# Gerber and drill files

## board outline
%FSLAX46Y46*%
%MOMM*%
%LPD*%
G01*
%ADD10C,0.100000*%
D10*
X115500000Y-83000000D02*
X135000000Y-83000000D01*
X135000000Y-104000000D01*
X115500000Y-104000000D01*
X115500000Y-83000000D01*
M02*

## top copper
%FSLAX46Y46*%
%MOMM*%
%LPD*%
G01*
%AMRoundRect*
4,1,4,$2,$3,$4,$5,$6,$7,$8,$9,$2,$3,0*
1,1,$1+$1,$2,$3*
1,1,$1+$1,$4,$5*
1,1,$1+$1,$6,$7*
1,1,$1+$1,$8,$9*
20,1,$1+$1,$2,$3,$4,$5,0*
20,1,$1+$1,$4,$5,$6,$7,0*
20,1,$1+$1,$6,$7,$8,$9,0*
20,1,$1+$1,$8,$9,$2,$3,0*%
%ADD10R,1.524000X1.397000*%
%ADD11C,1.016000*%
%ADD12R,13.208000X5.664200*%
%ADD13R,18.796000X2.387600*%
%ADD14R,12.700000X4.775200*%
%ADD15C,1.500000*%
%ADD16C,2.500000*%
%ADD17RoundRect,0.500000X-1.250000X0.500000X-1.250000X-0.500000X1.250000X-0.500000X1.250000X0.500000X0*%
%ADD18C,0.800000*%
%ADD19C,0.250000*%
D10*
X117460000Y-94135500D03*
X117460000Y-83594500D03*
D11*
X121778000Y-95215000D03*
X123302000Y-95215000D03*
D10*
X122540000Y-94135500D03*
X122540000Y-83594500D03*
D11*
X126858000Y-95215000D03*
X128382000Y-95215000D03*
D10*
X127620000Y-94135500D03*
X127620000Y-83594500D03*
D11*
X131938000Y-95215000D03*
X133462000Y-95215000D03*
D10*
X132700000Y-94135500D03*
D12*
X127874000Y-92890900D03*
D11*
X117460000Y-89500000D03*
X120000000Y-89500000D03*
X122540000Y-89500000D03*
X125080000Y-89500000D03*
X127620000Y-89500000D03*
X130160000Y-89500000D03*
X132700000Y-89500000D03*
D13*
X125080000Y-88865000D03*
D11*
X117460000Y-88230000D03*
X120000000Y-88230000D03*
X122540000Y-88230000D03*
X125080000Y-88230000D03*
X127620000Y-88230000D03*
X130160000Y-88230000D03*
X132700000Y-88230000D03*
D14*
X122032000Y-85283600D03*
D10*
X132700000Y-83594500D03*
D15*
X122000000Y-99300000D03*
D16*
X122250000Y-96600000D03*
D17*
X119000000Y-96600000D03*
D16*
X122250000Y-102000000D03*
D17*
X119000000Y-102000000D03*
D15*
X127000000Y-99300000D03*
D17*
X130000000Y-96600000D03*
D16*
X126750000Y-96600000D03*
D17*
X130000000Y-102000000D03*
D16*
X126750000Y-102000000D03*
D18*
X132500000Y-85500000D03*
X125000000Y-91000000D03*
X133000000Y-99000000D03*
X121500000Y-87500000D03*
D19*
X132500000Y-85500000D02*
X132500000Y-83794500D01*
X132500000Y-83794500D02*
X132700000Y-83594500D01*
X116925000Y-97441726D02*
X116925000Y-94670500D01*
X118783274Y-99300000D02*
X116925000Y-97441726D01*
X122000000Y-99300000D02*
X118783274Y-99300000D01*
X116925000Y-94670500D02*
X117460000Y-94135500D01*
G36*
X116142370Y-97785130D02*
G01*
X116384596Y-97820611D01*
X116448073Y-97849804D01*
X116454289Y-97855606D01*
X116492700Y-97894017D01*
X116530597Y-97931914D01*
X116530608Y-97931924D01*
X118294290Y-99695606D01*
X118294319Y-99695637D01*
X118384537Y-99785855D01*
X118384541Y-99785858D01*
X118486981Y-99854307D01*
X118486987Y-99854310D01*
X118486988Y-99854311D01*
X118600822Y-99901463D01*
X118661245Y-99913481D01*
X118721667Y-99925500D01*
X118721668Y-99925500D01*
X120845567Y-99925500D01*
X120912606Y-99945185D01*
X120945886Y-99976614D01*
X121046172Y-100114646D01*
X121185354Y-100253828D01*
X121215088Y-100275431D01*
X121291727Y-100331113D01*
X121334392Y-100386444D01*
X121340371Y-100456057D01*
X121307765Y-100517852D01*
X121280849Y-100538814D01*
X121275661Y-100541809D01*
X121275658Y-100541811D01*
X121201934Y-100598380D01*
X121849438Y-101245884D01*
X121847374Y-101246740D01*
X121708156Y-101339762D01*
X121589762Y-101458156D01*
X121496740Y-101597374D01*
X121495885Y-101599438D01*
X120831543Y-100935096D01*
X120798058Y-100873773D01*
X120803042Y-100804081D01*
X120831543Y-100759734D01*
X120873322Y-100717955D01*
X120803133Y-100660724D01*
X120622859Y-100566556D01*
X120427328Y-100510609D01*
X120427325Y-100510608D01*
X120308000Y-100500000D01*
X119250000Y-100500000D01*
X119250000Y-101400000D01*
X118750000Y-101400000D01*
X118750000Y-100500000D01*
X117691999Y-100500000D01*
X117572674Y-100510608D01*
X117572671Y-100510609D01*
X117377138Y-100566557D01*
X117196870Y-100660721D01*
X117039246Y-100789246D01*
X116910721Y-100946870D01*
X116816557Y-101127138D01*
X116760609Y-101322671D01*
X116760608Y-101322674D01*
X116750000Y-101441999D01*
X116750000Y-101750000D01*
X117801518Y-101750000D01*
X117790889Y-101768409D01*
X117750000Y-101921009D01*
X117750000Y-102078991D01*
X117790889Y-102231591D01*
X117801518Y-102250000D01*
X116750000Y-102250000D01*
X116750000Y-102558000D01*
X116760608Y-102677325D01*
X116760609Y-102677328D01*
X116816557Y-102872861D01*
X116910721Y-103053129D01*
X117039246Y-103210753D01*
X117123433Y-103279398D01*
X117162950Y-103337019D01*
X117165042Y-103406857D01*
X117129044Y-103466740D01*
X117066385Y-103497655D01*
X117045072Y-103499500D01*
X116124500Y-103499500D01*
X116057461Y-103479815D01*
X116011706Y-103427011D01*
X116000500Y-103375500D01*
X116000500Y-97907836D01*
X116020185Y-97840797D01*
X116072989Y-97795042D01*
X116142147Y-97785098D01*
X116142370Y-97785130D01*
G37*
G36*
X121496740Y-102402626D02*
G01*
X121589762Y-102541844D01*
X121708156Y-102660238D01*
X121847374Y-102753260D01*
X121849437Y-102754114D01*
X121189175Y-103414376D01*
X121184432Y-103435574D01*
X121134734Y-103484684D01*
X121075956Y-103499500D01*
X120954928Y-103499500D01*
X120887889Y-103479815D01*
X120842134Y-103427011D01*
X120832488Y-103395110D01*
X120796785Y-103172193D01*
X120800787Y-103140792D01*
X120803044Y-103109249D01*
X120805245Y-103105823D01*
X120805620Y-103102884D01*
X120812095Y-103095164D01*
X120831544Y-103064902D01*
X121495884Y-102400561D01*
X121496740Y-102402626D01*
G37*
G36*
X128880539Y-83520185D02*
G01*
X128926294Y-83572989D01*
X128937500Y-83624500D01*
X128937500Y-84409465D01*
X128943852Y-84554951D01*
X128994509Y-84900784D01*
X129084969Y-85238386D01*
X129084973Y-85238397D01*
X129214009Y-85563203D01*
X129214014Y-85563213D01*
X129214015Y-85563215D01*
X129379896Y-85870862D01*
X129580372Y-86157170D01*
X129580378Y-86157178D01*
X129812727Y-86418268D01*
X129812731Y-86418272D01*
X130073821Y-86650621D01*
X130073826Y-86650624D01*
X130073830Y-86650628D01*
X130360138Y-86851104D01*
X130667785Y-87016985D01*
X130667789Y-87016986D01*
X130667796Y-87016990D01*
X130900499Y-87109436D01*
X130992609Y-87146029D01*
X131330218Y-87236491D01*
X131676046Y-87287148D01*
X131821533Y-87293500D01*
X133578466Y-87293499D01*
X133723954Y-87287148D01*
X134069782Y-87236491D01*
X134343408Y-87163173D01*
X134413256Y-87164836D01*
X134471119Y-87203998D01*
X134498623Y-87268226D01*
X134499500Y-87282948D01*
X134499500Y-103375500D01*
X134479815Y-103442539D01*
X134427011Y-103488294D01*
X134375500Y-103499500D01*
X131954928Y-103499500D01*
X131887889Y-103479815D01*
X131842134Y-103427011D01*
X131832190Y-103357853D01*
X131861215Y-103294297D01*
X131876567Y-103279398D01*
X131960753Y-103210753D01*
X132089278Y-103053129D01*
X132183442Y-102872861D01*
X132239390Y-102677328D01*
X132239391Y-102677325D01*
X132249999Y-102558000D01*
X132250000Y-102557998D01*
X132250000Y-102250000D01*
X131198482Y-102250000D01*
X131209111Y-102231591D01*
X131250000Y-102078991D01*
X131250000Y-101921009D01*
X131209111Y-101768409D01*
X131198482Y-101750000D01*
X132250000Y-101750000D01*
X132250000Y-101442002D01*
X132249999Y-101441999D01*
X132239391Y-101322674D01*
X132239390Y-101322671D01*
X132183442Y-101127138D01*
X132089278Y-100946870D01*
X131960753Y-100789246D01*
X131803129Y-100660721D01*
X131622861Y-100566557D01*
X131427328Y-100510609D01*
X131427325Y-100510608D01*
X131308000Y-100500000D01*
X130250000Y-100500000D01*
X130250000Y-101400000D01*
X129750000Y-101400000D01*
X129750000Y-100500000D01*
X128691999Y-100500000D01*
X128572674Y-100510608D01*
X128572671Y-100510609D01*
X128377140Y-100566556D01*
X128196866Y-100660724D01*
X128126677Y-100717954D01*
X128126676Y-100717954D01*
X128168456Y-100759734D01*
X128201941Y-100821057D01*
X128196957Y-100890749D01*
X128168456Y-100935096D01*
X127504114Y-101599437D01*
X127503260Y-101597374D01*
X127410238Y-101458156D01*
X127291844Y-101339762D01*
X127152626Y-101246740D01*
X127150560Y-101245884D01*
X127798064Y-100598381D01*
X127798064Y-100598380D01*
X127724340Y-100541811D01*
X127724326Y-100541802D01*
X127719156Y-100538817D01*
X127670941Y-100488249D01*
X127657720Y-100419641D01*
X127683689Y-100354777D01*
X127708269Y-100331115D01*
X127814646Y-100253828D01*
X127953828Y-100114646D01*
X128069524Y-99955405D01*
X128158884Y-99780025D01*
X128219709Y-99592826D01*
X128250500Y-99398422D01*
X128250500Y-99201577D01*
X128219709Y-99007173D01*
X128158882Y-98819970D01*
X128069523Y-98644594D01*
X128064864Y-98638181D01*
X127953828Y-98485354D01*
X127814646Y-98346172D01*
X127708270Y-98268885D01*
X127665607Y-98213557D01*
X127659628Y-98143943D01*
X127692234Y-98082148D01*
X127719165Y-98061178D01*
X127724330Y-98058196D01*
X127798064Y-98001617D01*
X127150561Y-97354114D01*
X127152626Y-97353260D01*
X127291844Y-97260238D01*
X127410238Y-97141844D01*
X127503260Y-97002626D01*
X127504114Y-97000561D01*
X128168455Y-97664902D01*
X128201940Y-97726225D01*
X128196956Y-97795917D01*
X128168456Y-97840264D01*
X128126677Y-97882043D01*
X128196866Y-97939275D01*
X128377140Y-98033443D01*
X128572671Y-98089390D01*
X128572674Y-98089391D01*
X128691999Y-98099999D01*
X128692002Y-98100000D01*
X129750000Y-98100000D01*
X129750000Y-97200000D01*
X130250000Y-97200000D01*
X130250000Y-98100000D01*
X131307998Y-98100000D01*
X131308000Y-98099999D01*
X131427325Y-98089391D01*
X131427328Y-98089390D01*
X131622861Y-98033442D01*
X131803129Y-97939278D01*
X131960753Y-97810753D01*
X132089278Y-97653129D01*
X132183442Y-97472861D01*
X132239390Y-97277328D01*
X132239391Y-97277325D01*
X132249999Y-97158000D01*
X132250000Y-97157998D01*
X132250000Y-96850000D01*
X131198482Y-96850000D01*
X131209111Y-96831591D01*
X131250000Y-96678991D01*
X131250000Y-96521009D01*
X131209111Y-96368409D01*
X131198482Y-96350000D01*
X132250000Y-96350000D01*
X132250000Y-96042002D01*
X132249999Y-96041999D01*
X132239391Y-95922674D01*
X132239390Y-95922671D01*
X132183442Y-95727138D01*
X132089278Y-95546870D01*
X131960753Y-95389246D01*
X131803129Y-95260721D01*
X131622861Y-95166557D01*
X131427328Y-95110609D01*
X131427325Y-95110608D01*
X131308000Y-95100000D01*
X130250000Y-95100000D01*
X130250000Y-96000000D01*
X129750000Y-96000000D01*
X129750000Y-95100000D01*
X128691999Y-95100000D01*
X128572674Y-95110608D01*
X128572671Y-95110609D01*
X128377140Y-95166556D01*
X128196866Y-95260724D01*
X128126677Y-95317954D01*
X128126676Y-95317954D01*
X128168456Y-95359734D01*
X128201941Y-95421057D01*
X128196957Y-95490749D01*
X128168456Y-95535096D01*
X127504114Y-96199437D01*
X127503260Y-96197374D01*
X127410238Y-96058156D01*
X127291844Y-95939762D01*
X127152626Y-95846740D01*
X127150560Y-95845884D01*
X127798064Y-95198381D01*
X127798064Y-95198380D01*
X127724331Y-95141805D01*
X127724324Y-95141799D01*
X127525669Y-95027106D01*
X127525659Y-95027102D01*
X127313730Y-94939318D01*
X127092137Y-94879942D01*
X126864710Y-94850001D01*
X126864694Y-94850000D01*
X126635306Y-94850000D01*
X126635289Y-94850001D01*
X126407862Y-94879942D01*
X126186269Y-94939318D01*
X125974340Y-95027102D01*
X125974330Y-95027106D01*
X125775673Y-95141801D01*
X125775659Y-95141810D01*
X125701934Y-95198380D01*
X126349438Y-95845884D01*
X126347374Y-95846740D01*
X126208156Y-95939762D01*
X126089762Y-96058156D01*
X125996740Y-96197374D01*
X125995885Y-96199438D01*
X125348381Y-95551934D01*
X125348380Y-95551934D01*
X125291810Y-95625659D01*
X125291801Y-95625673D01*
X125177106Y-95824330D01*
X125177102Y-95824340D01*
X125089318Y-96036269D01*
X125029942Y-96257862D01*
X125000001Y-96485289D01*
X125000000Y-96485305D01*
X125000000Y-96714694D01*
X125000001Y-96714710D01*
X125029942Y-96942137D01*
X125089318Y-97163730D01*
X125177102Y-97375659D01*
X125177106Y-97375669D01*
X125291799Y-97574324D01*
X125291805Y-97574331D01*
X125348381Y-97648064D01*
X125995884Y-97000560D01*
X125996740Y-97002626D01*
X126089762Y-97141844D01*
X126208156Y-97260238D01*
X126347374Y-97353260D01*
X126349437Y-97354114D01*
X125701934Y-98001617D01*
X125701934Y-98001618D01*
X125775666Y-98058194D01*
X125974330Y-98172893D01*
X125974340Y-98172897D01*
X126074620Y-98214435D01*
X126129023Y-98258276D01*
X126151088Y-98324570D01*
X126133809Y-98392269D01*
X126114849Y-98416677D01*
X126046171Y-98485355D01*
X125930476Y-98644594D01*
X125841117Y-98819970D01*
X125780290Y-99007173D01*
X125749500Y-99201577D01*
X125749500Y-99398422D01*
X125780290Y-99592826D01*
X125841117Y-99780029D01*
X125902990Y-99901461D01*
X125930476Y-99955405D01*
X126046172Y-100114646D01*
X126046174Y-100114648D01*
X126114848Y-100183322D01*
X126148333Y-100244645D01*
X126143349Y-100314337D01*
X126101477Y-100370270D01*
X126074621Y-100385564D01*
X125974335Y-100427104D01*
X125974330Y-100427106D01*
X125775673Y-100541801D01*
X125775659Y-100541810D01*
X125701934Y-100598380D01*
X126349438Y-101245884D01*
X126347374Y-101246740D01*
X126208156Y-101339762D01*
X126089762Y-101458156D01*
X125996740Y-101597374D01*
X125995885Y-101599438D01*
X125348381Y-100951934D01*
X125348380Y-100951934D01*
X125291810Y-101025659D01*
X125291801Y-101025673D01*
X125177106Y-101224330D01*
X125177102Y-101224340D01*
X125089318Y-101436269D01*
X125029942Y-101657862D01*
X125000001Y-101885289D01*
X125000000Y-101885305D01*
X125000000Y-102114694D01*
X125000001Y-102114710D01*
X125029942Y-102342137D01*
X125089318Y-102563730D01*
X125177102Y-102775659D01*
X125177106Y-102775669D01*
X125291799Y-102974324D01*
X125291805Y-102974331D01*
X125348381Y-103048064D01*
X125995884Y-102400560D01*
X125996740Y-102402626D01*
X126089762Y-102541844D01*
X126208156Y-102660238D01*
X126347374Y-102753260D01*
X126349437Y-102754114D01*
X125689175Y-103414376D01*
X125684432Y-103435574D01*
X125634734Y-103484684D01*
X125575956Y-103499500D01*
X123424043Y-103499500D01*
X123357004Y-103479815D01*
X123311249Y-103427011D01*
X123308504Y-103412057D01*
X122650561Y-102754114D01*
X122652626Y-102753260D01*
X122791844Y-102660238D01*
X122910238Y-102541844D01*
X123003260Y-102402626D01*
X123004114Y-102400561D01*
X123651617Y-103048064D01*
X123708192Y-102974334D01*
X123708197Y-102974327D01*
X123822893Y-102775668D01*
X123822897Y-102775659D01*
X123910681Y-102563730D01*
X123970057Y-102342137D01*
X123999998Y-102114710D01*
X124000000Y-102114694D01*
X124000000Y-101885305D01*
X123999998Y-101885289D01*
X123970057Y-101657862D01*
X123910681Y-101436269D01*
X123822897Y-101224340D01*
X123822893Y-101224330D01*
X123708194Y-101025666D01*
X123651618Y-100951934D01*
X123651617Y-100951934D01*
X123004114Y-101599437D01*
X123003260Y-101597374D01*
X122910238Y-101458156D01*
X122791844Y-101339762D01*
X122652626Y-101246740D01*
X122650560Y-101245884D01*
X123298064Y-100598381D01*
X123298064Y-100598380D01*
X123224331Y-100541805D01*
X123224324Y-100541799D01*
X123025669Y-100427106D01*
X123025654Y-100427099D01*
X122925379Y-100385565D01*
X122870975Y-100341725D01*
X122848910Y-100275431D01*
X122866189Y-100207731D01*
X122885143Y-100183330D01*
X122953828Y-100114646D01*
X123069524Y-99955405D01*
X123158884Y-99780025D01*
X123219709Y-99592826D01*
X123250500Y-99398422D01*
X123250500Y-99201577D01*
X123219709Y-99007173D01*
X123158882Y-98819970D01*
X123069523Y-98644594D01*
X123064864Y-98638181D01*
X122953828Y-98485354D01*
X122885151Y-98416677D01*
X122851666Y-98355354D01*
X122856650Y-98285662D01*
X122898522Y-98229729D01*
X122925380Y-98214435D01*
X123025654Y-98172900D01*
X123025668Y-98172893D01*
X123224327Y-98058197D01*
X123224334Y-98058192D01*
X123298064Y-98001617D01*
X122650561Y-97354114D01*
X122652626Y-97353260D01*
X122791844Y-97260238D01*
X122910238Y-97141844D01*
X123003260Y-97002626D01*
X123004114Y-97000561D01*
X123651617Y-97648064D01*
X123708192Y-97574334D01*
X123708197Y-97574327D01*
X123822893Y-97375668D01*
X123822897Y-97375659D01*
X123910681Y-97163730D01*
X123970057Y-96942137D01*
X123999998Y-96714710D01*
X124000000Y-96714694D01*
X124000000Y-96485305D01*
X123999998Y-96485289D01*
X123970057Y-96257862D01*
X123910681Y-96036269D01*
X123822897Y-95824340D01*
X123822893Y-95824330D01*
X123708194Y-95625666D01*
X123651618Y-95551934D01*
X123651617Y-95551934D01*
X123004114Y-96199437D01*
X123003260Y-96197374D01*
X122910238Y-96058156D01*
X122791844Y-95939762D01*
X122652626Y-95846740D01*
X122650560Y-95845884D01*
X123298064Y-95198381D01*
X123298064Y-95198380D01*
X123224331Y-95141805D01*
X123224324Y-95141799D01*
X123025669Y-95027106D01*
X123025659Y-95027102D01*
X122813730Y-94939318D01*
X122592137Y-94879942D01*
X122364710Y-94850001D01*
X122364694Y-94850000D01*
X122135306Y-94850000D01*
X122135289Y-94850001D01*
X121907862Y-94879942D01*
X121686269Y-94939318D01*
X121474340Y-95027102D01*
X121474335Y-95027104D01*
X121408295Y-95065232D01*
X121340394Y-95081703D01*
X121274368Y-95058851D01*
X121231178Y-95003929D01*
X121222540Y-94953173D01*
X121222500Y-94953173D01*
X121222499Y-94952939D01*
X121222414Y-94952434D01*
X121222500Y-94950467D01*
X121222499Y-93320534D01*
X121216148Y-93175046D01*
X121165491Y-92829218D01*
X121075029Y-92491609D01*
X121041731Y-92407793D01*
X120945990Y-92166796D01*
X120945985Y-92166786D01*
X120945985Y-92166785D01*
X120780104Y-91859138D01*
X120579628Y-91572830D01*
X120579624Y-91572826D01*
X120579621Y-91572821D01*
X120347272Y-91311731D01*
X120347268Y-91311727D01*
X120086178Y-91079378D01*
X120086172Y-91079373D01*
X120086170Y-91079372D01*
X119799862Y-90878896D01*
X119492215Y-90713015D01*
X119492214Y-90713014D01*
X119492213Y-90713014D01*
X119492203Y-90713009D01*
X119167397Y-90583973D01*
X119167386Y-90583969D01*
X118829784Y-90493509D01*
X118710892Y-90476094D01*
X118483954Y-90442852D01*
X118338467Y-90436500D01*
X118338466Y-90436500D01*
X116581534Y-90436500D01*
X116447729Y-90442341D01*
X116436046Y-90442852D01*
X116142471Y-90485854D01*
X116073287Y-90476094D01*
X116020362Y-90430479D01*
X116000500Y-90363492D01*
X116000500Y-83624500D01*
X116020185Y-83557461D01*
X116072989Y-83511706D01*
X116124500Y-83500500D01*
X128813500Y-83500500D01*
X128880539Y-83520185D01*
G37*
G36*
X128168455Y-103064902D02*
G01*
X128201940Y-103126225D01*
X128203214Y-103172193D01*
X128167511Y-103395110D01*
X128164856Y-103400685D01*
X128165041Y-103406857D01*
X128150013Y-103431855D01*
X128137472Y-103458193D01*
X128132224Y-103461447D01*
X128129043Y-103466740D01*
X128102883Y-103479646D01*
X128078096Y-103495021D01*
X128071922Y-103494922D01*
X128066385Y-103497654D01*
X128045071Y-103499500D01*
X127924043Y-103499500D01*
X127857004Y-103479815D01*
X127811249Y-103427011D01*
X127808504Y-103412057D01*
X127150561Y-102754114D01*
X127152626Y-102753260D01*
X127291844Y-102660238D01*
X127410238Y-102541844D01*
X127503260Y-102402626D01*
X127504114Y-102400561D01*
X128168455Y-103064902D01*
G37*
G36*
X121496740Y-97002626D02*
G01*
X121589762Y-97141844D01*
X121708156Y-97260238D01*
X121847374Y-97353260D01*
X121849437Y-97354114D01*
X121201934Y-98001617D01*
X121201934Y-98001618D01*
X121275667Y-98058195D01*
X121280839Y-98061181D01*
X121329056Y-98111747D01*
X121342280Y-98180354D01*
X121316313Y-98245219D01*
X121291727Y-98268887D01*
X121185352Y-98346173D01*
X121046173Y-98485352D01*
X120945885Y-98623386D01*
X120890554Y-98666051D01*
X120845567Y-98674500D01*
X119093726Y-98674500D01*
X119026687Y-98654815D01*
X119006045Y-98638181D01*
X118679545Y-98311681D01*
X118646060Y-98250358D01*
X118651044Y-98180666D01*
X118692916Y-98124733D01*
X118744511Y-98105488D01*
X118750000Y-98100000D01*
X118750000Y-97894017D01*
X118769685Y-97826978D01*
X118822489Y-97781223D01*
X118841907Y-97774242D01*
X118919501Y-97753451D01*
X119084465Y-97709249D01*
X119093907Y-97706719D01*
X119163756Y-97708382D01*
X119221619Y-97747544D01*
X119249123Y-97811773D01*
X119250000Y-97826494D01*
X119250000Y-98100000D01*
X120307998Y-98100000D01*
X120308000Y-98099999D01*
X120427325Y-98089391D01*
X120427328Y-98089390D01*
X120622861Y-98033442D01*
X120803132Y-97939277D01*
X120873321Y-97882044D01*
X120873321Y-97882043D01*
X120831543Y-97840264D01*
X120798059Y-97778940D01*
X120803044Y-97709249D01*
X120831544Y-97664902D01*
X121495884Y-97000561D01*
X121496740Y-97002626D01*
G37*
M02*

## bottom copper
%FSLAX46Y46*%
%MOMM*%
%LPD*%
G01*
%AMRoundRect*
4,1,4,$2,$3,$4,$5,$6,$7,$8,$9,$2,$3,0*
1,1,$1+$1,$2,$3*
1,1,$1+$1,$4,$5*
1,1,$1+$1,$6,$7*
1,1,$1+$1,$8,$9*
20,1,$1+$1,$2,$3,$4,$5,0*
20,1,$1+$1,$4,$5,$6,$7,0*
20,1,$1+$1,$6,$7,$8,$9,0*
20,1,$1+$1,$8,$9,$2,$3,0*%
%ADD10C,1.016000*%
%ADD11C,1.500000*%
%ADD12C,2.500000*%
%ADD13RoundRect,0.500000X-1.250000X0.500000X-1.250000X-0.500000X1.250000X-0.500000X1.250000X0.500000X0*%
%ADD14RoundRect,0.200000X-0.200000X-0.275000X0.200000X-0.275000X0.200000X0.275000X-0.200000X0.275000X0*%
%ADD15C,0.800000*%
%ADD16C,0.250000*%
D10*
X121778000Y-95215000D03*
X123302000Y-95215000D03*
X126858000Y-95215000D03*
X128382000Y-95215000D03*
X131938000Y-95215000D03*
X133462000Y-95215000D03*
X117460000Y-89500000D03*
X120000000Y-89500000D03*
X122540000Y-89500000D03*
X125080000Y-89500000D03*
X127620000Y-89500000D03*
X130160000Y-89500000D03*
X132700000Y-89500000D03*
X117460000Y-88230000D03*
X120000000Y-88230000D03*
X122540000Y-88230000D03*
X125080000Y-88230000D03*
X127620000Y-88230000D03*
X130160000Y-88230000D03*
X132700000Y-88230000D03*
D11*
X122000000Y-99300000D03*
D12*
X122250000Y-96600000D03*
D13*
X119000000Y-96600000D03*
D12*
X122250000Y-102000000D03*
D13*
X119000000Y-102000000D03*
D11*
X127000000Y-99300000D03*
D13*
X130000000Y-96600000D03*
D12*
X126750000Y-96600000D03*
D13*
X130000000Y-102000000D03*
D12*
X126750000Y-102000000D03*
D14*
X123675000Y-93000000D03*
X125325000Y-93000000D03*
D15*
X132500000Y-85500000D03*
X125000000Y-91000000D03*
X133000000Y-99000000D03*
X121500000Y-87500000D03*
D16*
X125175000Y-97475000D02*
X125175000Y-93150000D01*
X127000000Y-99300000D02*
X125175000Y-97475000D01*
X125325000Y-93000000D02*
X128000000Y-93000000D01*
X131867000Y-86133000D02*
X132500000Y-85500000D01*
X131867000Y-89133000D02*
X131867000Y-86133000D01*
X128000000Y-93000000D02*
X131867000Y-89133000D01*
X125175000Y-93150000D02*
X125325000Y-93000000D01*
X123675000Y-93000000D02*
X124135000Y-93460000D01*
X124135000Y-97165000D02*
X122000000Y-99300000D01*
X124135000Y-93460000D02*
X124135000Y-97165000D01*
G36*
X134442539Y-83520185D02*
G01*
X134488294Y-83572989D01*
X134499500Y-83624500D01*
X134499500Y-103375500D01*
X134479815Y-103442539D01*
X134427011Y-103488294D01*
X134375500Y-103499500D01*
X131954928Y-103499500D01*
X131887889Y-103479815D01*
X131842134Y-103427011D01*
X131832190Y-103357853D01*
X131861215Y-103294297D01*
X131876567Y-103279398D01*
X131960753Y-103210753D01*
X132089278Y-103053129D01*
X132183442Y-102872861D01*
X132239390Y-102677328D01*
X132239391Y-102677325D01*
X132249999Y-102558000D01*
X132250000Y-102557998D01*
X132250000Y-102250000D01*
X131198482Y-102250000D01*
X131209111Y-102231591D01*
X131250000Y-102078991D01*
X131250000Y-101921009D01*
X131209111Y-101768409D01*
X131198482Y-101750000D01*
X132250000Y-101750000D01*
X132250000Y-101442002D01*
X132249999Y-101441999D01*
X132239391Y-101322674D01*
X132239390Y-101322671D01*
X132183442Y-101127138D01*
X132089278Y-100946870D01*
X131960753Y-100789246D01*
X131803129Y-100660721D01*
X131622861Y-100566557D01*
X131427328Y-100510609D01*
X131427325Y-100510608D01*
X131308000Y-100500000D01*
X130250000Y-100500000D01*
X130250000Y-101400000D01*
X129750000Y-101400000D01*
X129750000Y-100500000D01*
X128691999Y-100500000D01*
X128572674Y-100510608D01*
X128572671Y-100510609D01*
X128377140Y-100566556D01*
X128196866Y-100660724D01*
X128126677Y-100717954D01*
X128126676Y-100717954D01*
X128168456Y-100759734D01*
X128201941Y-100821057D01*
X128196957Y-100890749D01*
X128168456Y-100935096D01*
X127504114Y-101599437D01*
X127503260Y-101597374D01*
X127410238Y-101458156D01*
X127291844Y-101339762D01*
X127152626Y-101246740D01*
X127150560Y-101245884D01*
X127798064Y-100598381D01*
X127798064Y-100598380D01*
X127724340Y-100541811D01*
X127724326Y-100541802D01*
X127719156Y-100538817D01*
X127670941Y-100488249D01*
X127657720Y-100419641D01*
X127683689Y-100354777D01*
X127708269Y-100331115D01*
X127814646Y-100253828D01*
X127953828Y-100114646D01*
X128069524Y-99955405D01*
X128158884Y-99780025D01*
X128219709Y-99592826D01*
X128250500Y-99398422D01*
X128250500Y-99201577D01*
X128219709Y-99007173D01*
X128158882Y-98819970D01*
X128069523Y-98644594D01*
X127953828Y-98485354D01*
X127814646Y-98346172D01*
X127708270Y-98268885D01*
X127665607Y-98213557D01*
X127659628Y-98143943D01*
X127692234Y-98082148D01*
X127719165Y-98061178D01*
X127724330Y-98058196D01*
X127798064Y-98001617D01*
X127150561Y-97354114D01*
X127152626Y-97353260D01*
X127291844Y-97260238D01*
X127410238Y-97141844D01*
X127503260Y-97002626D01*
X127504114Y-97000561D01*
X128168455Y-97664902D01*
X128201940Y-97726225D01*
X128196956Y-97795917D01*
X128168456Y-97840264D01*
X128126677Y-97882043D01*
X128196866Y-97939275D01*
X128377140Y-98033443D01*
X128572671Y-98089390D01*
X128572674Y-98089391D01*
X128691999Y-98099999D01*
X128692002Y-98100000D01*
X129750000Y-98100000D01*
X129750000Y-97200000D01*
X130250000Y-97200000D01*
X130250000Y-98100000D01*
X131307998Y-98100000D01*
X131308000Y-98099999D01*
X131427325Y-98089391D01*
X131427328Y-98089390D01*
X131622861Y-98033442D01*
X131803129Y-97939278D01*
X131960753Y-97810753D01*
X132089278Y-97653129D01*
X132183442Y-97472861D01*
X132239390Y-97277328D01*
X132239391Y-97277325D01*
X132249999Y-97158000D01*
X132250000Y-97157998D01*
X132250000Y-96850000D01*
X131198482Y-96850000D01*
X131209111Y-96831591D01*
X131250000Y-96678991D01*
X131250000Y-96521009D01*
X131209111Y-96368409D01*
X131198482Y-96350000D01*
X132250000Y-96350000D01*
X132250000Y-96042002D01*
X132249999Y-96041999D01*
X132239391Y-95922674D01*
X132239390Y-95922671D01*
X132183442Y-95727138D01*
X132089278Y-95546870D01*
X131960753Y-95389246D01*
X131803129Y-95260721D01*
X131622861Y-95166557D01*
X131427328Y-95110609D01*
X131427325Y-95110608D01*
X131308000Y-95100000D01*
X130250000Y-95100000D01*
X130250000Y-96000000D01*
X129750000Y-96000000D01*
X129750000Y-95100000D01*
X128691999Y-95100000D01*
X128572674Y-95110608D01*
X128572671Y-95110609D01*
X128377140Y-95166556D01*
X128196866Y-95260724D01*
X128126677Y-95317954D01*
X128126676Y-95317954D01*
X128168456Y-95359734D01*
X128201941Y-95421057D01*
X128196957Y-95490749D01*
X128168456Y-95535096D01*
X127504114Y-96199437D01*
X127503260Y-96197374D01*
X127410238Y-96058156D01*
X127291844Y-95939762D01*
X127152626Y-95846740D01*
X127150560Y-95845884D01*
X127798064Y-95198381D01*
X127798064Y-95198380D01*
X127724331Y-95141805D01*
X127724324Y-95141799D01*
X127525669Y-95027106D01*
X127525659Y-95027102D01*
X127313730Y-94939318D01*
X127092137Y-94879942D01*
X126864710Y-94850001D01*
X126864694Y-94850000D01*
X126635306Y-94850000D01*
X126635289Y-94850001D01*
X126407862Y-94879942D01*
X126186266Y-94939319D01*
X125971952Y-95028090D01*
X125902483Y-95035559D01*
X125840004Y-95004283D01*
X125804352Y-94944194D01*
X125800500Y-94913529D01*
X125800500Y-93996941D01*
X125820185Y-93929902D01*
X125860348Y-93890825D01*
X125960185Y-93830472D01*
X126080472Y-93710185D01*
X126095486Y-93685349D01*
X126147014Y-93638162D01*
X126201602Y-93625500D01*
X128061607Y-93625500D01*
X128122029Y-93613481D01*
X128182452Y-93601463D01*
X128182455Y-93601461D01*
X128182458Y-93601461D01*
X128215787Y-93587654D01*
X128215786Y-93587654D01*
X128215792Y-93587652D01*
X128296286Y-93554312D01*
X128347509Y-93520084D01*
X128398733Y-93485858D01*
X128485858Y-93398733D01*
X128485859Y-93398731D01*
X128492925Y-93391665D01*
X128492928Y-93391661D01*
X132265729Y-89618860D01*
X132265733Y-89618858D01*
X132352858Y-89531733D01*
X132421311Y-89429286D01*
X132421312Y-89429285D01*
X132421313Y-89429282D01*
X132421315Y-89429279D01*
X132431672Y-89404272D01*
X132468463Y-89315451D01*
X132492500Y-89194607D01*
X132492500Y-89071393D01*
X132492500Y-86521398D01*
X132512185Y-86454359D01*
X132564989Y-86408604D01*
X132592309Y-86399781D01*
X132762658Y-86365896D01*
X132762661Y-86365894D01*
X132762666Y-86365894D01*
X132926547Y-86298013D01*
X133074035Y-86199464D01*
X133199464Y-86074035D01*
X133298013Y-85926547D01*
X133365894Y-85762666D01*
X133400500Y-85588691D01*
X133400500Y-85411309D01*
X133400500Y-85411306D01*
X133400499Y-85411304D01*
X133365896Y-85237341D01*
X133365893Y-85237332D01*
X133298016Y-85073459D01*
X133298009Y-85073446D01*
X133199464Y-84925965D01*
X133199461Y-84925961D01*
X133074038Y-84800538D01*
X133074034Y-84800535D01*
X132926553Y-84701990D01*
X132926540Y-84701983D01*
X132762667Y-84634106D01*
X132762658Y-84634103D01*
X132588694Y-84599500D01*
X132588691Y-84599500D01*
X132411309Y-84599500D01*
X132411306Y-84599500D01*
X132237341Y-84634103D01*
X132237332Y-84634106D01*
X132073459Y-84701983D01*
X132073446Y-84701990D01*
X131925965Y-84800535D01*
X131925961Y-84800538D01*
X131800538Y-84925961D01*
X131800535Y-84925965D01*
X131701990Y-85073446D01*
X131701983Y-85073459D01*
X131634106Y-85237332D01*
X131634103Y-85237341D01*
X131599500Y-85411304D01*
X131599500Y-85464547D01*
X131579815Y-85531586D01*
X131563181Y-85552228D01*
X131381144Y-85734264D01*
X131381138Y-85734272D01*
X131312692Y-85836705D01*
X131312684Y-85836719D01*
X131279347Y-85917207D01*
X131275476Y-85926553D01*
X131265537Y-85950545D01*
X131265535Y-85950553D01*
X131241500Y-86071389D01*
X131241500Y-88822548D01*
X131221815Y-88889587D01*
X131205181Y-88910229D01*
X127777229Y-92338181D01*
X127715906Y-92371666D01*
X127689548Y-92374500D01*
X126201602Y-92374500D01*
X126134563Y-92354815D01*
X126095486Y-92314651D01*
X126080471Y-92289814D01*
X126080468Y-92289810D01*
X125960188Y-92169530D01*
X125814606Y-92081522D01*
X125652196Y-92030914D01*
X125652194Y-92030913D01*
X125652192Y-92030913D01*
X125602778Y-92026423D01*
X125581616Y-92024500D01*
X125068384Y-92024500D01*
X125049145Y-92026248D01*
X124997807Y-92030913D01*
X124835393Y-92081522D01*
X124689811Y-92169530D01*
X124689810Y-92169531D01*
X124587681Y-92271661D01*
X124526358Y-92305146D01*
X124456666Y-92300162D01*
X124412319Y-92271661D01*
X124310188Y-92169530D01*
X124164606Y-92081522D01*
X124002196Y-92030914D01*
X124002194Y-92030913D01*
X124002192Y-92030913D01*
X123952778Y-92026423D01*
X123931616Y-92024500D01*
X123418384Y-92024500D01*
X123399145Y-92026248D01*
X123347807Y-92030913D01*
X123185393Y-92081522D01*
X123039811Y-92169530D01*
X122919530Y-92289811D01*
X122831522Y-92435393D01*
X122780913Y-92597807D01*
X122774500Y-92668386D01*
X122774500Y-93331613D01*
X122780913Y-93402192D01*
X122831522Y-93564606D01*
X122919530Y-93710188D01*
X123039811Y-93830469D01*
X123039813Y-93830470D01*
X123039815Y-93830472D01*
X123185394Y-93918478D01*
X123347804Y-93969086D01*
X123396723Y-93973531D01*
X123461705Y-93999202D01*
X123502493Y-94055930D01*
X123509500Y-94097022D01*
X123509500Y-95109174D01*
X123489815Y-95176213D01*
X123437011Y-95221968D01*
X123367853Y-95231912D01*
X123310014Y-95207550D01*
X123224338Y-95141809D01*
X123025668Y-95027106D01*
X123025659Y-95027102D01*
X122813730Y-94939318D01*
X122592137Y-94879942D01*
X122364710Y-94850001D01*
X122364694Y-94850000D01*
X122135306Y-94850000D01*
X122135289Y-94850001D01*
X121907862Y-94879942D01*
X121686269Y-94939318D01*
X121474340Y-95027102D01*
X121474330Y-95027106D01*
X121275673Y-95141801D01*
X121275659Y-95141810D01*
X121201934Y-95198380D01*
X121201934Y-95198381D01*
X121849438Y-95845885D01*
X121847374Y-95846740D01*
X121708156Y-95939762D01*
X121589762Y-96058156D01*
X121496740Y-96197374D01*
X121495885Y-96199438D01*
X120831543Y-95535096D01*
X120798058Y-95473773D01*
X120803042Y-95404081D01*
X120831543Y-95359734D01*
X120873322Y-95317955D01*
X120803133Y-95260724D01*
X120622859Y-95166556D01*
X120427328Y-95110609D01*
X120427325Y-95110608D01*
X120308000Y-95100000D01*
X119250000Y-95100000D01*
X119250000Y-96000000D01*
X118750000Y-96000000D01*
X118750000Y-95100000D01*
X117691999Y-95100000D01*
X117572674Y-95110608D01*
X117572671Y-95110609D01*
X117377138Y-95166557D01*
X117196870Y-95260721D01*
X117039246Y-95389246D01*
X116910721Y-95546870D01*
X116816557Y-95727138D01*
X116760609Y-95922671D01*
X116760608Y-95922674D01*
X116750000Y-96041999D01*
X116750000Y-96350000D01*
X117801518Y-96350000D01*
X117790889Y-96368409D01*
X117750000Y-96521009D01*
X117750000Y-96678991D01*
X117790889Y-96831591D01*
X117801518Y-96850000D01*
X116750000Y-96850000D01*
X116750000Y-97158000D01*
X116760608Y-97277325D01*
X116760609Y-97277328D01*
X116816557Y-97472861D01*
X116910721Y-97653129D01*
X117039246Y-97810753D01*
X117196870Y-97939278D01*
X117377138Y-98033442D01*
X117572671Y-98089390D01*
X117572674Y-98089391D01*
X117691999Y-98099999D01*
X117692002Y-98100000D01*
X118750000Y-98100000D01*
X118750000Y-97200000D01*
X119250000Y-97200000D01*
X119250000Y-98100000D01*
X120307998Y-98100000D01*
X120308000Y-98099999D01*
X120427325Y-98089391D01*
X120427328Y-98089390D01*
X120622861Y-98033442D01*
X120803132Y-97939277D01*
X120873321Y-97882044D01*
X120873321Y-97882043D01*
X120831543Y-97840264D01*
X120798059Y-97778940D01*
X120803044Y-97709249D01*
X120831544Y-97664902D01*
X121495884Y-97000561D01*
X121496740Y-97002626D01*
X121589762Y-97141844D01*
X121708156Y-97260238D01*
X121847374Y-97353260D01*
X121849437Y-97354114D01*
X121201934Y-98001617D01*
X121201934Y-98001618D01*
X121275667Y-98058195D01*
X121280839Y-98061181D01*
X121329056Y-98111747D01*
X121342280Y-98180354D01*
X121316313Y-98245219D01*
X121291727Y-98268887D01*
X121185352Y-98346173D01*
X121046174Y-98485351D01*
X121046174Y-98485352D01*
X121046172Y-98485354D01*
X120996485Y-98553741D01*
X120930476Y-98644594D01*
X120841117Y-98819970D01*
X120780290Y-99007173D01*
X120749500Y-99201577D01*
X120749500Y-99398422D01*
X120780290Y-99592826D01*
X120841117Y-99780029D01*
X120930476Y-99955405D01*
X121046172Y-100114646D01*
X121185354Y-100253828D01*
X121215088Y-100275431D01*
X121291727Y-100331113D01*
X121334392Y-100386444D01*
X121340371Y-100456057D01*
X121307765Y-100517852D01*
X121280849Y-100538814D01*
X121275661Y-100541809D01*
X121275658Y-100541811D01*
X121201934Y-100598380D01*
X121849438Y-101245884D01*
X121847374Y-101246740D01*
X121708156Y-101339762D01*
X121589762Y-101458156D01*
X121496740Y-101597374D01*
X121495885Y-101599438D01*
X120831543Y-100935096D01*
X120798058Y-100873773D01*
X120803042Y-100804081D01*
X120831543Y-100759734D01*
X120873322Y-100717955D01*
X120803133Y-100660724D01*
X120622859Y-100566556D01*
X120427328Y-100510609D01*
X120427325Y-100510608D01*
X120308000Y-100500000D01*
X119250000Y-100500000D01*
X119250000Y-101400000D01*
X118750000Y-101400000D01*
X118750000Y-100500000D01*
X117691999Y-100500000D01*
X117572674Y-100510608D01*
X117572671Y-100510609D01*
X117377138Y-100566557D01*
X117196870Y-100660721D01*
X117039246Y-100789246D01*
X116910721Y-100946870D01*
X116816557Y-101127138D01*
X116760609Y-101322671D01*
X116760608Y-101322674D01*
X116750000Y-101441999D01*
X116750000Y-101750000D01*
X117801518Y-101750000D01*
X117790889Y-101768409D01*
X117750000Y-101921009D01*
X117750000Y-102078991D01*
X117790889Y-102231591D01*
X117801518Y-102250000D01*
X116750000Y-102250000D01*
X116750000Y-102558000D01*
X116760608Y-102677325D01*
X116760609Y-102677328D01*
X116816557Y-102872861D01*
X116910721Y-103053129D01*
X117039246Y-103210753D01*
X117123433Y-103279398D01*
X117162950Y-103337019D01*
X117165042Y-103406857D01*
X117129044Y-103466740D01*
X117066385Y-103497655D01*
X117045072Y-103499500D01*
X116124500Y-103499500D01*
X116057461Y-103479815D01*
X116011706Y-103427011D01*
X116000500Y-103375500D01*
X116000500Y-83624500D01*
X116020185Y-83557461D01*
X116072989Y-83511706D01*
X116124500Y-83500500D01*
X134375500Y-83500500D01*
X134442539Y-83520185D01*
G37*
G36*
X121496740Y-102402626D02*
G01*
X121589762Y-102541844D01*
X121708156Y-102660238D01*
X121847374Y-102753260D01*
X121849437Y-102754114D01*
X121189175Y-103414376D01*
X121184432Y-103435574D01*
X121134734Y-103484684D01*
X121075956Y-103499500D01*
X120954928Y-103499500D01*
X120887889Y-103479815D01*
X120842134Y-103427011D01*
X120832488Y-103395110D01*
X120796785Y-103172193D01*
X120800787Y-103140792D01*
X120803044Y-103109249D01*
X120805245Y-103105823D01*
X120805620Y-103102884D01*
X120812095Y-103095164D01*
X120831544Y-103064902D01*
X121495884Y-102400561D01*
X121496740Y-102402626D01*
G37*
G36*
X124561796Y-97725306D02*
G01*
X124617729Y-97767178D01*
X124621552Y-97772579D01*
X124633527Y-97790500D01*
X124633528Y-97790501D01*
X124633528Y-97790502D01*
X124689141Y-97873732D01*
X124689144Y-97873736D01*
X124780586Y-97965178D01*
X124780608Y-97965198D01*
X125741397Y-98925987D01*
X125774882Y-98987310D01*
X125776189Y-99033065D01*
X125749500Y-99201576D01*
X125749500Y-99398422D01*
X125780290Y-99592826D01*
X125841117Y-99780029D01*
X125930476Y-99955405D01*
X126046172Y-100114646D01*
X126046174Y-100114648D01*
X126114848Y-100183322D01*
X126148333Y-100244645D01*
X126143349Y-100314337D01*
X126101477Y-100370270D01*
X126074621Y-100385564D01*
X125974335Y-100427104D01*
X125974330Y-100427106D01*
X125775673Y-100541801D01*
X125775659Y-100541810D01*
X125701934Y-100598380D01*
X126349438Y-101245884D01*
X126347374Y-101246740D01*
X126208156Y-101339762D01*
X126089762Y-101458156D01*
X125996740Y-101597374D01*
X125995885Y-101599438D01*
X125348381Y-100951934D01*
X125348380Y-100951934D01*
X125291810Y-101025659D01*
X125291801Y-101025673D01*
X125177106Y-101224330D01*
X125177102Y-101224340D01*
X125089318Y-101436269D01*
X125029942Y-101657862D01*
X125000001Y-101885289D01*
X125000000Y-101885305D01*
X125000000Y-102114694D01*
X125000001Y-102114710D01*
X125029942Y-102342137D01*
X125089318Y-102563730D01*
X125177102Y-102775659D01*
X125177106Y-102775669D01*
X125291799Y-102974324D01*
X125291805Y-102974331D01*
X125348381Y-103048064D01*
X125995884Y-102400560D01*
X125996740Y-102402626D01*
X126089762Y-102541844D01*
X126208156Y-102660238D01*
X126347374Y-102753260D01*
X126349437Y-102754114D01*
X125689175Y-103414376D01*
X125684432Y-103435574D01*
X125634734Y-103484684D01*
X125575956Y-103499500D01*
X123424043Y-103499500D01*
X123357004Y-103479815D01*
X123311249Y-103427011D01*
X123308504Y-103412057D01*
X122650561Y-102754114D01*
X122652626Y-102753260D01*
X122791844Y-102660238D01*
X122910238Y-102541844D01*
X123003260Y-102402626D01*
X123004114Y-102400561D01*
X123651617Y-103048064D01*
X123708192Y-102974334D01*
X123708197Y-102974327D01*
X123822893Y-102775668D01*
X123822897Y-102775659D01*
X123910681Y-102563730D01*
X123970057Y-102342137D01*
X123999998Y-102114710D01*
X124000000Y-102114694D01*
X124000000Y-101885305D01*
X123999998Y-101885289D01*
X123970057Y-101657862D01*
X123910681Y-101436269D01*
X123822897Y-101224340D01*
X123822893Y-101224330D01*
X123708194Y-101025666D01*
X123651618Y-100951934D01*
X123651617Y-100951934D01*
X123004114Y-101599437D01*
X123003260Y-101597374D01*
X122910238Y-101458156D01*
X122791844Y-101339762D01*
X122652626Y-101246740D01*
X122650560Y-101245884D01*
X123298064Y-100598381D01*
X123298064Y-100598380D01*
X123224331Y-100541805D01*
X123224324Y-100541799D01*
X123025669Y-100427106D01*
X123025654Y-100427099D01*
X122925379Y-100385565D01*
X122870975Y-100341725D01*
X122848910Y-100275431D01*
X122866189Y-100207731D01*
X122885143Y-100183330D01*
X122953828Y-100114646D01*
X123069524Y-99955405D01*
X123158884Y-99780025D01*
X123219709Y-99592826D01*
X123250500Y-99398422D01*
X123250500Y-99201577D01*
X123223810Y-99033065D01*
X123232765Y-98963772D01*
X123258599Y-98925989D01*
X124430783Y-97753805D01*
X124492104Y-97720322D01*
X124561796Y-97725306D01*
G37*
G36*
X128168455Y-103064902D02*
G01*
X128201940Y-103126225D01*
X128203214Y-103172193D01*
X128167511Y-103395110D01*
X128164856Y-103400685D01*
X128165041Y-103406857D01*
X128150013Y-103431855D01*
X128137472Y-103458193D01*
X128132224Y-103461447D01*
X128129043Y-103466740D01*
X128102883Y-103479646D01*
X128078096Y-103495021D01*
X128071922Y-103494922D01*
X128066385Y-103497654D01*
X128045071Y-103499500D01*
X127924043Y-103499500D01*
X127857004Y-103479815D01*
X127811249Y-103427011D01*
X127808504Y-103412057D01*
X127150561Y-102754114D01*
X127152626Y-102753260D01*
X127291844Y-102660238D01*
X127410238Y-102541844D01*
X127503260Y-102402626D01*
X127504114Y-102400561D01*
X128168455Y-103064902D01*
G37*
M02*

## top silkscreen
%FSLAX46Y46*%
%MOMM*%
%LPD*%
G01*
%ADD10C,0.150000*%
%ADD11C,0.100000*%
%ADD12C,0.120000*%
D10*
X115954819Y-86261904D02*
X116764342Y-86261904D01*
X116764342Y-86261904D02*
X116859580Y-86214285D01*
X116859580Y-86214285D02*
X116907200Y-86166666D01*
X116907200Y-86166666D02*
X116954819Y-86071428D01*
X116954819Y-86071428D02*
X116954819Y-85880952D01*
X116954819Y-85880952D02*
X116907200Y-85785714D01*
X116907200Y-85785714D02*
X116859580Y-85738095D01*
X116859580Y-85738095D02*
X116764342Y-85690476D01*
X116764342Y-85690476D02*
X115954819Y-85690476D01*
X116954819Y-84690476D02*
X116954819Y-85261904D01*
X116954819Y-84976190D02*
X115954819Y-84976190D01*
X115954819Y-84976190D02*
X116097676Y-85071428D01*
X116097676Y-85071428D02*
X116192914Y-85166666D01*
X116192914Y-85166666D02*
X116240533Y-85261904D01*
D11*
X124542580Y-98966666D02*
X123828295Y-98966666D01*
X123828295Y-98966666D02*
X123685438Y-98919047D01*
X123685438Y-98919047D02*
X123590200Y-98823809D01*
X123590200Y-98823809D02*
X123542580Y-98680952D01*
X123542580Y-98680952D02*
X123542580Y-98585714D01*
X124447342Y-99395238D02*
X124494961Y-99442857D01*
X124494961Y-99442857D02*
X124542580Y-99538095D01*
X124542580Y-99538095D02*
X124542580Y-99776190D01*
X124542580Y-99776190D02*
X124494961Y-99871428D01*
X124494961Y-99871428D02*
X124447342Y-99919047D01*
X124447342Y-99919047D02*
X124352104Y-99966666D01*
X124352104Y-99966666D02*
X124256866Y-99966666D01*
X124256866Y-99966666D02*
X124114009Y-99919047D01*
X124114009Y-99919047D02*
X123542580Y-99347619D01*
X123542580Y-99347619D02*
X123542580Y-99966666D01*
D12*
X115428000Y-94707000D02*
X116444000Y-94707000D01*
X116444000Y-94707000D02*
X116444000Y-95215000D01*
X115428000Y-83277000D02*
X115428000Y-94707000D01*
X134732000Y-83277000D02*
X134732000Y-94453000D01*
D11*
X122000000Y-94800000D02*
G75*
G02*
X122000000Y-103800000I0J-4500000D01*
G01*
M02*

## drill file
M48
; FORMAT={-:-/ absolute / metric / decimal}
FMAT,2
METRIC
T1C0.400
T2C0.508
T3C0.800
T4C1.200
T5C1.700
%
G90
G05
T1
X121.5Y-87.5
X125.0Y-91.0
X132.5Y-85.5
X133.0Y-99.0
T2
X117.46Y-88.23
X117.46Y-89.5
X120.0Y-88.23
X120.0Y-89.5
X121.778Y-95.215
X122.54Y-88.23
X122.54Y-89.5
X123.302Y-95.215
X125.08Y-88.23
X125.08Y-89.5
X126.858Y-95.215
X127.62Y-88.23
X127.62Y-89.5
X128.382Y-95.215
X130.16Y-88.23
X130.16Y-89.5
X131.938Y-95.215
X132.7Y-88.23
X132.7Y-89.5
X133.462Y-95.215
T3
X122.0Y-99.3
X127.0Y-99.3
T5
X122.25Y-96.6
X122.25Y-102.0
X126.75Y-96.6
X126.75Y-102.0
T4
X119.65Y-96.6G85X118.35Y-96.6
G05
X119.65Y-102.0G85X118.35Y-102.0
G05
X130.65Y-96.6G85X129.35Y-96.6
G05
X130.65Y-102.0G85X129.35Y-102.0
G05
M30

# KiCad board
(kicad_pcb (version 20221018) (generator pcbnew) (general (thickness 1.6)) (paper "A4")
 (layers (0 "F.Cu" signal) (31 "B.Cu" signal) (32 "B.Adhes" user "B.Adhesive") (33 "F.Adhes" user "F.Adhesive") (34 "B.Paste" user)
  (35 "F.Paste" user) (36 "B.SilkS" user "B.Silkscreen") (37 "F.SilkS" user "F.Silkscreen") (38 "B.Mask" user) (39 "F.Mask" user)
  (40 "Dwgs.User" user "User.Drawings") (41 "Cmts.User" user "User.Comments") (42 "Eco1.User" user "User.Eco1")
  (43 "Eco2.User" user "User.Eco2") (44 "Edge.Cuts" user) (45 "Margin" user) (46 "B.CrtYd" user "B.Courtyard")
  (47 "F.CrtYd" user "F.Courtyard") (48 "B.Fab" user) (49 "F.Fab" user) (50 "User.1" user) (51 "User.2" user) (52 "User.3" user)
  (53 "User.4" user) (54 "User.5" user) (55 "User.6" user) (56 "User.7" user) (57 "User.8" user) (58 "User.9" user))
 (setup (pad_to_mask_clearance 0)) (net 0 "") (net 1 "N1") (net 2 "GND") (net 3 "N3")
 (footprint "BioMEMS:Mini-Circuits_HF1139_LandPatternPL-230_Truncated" (layer "F.Cu") (at 125.08 88.865 90)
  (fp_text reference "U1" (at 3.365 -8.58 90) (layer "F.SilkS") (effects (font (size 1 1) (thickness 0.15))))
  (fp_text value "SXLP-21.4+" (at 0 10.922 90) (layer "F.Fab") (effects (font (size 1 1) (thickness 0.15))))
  (fp_line (start -5.842 -9.652) (end -5.842 -8.636) (stroke (width 0.12) (type solid)) (layer "F.SilkS"))
  (fp_line (start -5.842 -8.636) (end -6.35 -8.636) (stroke (width 0.12) (type solid)) (layer "F.SilkS"))
  (fp_line (start 5.588 -9.652) (end -5.842 -9.652) (stroke (width 0.12) (type solid)) (layer "F.SilkS"))
  (fp_line (start 5.588 9.652) (end -5.588 9.652) (stroke (width 0.12) (type solid)) (layer "F.SilkS"))
  (pad "1" smd rect (at -5.2705 -7.62) (size 1.524 1.397) (layers "F.Cu" "F.Paste" "F.Mask") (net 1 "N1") (clearance 3))
  (pad "2" smd rect (at 5.2705 -7.62) (size 1.524 1.397) (layers "F.Cu" "F.Paste" "F.Mask") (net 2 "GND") (zone_connect 2))
  (pad "3" thru_hole circle (at -6.35 -3.302) (size 1.016 1.016) (drill 0.508) (layers "*.Cu") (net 2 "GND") (zone_connect 2))
  (pad "3" thru_hole circle (at -6.35 -1.778) (size 1.016 1.016) (drill 0.508) (layers "*.Cu") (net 2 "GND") (zone_connect 2))
  (pad "3" smd rect (at -5.2705 -2.54) (size 1.524 1.397) (layers "F.Cu" "F.Paste" "F.Mask") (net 2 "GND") (zone_connect 2))
  (pad "4" smd rect (at 5.2705 -2.54) (size 1.524 1.397) (layers "F.Cu" "F.Paste" "F.Mask") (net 2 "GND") (zone_connect 2))
  (pad "5" thru_hole circle (at -6.35 1.778) (size 1.016 1.016) (drill 0.508) (layers "*.Cu") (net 2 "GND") (zone_connect 2))
  (pad "5" thru_hole circle (at -6.35 3.302) (size 1.016 1.016) (drill 0.508) (layers "*.Cu") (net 2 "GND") (zone_connect 2))
  (pad "5" smd rect (at -5.2705 2.54) (size 1.524 1.397) (layers "F.Cu" "F.Paste" "F.Mask") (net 2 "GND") (zone_connect 2))
  (pad "6" smd rect (at 5.2705 2.54) (size 1.524 1.397) (layers "F.Cu" "F.Paste" "F.Mask") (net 2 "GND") (zone_connect 2))
  (pad "7" thru_hole circle (at -6.35 6.858) (size 1.016 1.016) (drill 0.508) (layers "*.Cu") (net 2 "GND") (zone_connect 2))
  (pad "7" thru_hole circle (at -6.35 8.382) (size 1.016 1.016) (drill 0.508) (layers "*.Cu") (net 2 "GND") (zone_connect 2))
  (pad "7" smd rect (at -5.2705 7.62) (size 1.524 1.397) (layers "F.Cu" "F.Paste" "F.Mask") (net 2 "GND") (zone_connect 2))
  (pad "7" smd rect (at -4.0259 2.794) (size 13.208 5.6642) (layers "F.Cu") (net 2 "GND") (zone_connect 2))
  (pad "7" thru_hole circle (at -0.635 -7.62) (size 1.016 1.016) (drill 0.508) (layers "*.Cu") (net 2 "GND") (zone_connect 2))
  (pad "7" thru_hole circle (at -0.635 -5.08) (size 1.016 1.016) (drill 0.508) (layers "*.Cu") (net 2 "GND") (zone_connect 2))
  (pad "7" thru_hole circle (at -0.635 -2.54) (size 1.016 1.016) (drill 0.508) (layers "*.Cu") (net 2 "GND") (zone_connect 2))
  (pad "7" thru_hole circle (at -0.635 0) (size 1.016 1.016) (drill 0.508) (layers "*.Cu") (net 2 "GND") (zone_connect 2))
  (pad "7" thru_hole circle (at -0.635 2.54) (size 1.016 1.016) (drill 0.508) (layers "*.Cu") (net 2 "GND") (zone_connect 2))
  (pad "7" thru_hole circle (at -0.635 5.08) (size 1.016 1.016) (drill 0.508) (layers "*.Cu") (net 2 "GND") (zone_connect 2))
  (pad "7" thru_hole circle (at -0.635 7.62) (size 1.016 1.016) (drill 0.508) (layers "*.Cu") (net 2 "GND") (zone_connect 2))
  (pad "7" smd rect (at 0 0) (size 18.796 2.3876) (layers "F.Cu") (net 2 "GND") (zone_connect 2))
  (pad "7" thru_hole circle (at 0.635 -7.62) (size 1.016 1.016) (drill 0.508) (layers "*.Cu") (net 2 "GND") (zone_connect 2))
  (pad "7" thru_hole circle (at 0.635 -5.08) (size 1.016 1.016) (drill 0.508) (layers "*.Cu") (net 2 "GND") (zone_connect 2))
  (pad "7" thru_hole circle (at 0.635 -2.54) (size 1.016 1.016) (drill 0.508) (layers "*.Cu") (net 2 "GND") (zone_connect 2))
  (pad "7" thru_hole circle (at 0.635 0) (size 1.016 1.016) (drill 0.508) (layers "*.Cu") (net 2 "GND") (zone_connect 2))
  (pad "7" thru_hole circle (at 0.635 2.54) (size 1.016 1.016) (drill 0.508) (layers "*.Cu") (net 2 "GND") (zone_connect 2))
  (pad "7" thru_hole circle (at 0.635 5.08) (size 1.016 1.016) (drill 0.508) (layers "*.Cu") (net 2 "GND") (zone_connect 2))
  (pad "7" thru_hole circle (at 0.635 7.62) (size 1.016 1.016) (drill 0.508) (layers "*.Cu") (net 2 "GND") (zone_connect 2))
  (pad "7" smd rect (at 3.5814 -3.048) (size 12.7 4.7752) (layers "F.Cu") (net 2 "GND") (zone_connect 2))
  (pad "8" smd rect (at 5.2705 7.62) (size 1.524 1.397) (layers "F.Cu" "F.Paste" "F.Mask") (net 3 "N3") (clearance 3)))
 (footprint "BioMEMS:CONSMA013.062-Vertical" (layer "F.Cu") (at 122 99.3 -90)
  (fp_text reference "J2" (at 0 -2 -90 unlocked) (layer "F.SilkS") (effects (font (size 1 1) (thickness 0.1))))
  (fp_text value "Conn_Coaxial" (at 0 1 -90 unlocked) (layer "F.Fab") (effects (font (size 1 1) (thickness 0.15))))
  (fp_arc (start -4.5 0) (mid 0 -4.5) (end 4.5 0) (stroke (width 0.1) (type default)) (layer "F.SilkS"))
  (pad "1" thru_hole circle (at 0 0 270) (size 1.5 1.5) (drill 0.8) (layers "*.Cu" "*.Mask") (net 1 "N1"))
  (pad "2" thru_hole circle (at -2.7 -0.25 270) (size 2.5 2.5) (drill 1.7) (layers "*.Cu" "*.Mask") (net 2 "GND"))
  (pad "2" thru_hole roundrect (at -2.7 3 270) (size 2 3.5) (drill oval 1.2 2.5) (layers "*.Cu" "*.Mask") (roundrect_rratio 0.25)
   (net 2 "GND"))
  (pad "2" thru_hole circle (at 2.7 -0.25 270) (size 2.5 2.5) (drill 1.7) (layers "*.Cu" "*.Mask") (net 2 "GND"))
  (pad "2" thru_hole roundrect (at 2.7 3 270) (size 2 3.5) (drill oval 1.2 2.5) (layers "*.Cu" "*.Mask") (roundrect_rratio 0.25)
   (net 2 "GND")))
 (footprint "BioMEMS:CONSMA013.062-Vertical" (layer "B.Cu") (at 127 99.3 -90)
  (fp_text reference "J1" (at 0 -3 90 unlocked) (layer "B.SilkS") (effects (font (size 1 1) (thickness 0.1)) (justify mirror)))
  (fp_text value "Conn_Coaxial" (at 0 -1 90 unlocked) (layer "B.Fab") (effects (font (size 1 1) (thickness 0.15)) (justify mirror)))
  (pad "1" thru_hole circle (at 0 0 270) (size 1.5 1.5) (drill 0.8) (layers "*.Cu" "*.Mask") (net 3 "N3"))
  (pad "2" thru_hole roundrect (at -2.7 -3 270) (size 2 3.5) (drill oval 1.2 2.5) (layers "*.Cu" "*.Mask") (roundrect_rratio 0.25)
   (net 2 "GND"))
  (pad "2" thru_hole circle (at -2.7 0.25 270) (size 2.5 2.5) (drill 1.7) (layers "*.Cu" "*.Mask") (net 2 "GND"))
  (pad "2" thru_hole roundrect (at 2.7 -3 270) (size 2 3.5) (drill oval 1.2 2.5) (layers "*.Cu" "*.Mask") (roundrect_rratio 0.25)
   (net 2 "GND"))
  (pad "2" thru_hole circle (at 2.7 0.25 270) (size 2.5 2.5) (drill 1.7) (layers "*.Cu" "*.Mask") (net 2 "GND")))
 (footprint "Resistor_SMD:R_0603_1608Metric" (layer "B.Cu") (at 124.5 93)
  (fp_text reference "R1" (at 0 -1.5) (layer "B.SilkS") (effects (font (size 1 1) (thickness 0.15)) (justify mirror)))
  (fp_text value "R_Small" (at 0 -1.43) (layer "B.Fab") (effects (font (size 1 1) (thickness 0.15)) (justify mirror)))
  (pad "1" smd roundrect (at -0.825 0) (size 0.8 0.95) (layers "B.Cu" "B.Paste" "B.Mask") (roundrect_rratio 0.25) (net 1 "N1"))
  (pad "2" smd roundrect (at 0.825 0) (size 0.8 0.95) (layers "B.Cu" "B.Paste" "B.Mask") (roundrect_rratio 0.25) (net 3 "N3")))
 (gr_rect (start 115.5 83) (end 135 104) (stroke (width 0.1) (type default)) (fill none) (layer "Edge.Cuts"))
 (segment (start 132.5 85.5) (end 132.5 83.7945) (width 0.25) (layer "F.Cu") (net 3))
 (segment (start 132.5 83.7945) (end 132.7 83.5945) (width 0.25) (layer "F.Cu") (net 3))
 (via (at 132.5 85.5) (size 0.8) (drill 0.4) (layers "F.Cu" "B.Cu") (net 3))
 (segment (start 125.175 97.475) (end 125.175 93.15) (width 0.25) (layer "B.Cu") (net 3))
 (segment (start 127 99.3) (end 125.175 97.475) (width 0.25) (layer "B.Cu") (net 3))
 (segment (start 125.325 93) (end 128 93) (width 0.25) (layer "B.Cu") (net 3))
 (segment (start 131.867 86.133) (end 132.5 85.5) (width 0.25) (layer "B.Cu") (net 3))
 (segment (start 131.867 89.133) (end 131.867 86.133) (width 0.25) (layer "B.Cu") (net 3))
 (segment (start 128 93) (end 131.867 89.133) (width 0.25) (layer "B.Cu") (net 3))
 (segment (start 125.175 93.15) (end 125.325 93) (width 0.25) (layer "B.Cu") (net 3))
 (via (at 125 91) (size 0.8) (drill 0.4) (layers "F.Cu" "B.Cu") (free) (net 2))
 (via (at 133 99) (size 0.8) (drill 0.4) (layers "F.Cu" "B.Cu") (free) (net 2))
 (via (at 121.5 87.5) (size 0.8) (drill 0.4) (layers "F.Cu" "B.Cu") (free) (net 2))
 (segment (start 116.925 97.441726) (end 116.925 94.6705) (width 0.25) (layer "F.Cu") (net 1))
 (segment (start 118.783274 99.3) (end 116.925 97.441726) (width 0.25) (layer "F.Cu") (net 1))
 (segment (start 122 99.3) (end 118.783274 99.3) (width 0.25) (layer "F.Cu") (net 1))
 (segment (start 116.925 94.6705) (end 117.46 94.1355) (width 0.25) (layer "F.Cu") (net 1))
 (segment (start 123.675 93) (end 124.135 93.46) (width 0.25) (layer "B.Cu") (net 1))
 (segment (start 124.135 97.165) (end 122 99.3) (width 0.25) (layer "B.Cu") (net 1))
 (segment (start 124.135 93.46) (end 124.135 97.165) (width 0.25) (layer "B.Cu") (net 1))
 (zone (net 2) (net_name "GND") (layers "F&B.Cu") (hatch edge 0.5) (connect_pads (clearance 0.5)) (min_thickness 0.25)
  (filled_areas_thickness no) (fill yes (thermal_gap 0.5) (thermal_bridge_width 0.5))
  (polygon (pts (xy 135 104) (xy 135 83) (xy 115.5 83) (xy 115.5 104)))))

